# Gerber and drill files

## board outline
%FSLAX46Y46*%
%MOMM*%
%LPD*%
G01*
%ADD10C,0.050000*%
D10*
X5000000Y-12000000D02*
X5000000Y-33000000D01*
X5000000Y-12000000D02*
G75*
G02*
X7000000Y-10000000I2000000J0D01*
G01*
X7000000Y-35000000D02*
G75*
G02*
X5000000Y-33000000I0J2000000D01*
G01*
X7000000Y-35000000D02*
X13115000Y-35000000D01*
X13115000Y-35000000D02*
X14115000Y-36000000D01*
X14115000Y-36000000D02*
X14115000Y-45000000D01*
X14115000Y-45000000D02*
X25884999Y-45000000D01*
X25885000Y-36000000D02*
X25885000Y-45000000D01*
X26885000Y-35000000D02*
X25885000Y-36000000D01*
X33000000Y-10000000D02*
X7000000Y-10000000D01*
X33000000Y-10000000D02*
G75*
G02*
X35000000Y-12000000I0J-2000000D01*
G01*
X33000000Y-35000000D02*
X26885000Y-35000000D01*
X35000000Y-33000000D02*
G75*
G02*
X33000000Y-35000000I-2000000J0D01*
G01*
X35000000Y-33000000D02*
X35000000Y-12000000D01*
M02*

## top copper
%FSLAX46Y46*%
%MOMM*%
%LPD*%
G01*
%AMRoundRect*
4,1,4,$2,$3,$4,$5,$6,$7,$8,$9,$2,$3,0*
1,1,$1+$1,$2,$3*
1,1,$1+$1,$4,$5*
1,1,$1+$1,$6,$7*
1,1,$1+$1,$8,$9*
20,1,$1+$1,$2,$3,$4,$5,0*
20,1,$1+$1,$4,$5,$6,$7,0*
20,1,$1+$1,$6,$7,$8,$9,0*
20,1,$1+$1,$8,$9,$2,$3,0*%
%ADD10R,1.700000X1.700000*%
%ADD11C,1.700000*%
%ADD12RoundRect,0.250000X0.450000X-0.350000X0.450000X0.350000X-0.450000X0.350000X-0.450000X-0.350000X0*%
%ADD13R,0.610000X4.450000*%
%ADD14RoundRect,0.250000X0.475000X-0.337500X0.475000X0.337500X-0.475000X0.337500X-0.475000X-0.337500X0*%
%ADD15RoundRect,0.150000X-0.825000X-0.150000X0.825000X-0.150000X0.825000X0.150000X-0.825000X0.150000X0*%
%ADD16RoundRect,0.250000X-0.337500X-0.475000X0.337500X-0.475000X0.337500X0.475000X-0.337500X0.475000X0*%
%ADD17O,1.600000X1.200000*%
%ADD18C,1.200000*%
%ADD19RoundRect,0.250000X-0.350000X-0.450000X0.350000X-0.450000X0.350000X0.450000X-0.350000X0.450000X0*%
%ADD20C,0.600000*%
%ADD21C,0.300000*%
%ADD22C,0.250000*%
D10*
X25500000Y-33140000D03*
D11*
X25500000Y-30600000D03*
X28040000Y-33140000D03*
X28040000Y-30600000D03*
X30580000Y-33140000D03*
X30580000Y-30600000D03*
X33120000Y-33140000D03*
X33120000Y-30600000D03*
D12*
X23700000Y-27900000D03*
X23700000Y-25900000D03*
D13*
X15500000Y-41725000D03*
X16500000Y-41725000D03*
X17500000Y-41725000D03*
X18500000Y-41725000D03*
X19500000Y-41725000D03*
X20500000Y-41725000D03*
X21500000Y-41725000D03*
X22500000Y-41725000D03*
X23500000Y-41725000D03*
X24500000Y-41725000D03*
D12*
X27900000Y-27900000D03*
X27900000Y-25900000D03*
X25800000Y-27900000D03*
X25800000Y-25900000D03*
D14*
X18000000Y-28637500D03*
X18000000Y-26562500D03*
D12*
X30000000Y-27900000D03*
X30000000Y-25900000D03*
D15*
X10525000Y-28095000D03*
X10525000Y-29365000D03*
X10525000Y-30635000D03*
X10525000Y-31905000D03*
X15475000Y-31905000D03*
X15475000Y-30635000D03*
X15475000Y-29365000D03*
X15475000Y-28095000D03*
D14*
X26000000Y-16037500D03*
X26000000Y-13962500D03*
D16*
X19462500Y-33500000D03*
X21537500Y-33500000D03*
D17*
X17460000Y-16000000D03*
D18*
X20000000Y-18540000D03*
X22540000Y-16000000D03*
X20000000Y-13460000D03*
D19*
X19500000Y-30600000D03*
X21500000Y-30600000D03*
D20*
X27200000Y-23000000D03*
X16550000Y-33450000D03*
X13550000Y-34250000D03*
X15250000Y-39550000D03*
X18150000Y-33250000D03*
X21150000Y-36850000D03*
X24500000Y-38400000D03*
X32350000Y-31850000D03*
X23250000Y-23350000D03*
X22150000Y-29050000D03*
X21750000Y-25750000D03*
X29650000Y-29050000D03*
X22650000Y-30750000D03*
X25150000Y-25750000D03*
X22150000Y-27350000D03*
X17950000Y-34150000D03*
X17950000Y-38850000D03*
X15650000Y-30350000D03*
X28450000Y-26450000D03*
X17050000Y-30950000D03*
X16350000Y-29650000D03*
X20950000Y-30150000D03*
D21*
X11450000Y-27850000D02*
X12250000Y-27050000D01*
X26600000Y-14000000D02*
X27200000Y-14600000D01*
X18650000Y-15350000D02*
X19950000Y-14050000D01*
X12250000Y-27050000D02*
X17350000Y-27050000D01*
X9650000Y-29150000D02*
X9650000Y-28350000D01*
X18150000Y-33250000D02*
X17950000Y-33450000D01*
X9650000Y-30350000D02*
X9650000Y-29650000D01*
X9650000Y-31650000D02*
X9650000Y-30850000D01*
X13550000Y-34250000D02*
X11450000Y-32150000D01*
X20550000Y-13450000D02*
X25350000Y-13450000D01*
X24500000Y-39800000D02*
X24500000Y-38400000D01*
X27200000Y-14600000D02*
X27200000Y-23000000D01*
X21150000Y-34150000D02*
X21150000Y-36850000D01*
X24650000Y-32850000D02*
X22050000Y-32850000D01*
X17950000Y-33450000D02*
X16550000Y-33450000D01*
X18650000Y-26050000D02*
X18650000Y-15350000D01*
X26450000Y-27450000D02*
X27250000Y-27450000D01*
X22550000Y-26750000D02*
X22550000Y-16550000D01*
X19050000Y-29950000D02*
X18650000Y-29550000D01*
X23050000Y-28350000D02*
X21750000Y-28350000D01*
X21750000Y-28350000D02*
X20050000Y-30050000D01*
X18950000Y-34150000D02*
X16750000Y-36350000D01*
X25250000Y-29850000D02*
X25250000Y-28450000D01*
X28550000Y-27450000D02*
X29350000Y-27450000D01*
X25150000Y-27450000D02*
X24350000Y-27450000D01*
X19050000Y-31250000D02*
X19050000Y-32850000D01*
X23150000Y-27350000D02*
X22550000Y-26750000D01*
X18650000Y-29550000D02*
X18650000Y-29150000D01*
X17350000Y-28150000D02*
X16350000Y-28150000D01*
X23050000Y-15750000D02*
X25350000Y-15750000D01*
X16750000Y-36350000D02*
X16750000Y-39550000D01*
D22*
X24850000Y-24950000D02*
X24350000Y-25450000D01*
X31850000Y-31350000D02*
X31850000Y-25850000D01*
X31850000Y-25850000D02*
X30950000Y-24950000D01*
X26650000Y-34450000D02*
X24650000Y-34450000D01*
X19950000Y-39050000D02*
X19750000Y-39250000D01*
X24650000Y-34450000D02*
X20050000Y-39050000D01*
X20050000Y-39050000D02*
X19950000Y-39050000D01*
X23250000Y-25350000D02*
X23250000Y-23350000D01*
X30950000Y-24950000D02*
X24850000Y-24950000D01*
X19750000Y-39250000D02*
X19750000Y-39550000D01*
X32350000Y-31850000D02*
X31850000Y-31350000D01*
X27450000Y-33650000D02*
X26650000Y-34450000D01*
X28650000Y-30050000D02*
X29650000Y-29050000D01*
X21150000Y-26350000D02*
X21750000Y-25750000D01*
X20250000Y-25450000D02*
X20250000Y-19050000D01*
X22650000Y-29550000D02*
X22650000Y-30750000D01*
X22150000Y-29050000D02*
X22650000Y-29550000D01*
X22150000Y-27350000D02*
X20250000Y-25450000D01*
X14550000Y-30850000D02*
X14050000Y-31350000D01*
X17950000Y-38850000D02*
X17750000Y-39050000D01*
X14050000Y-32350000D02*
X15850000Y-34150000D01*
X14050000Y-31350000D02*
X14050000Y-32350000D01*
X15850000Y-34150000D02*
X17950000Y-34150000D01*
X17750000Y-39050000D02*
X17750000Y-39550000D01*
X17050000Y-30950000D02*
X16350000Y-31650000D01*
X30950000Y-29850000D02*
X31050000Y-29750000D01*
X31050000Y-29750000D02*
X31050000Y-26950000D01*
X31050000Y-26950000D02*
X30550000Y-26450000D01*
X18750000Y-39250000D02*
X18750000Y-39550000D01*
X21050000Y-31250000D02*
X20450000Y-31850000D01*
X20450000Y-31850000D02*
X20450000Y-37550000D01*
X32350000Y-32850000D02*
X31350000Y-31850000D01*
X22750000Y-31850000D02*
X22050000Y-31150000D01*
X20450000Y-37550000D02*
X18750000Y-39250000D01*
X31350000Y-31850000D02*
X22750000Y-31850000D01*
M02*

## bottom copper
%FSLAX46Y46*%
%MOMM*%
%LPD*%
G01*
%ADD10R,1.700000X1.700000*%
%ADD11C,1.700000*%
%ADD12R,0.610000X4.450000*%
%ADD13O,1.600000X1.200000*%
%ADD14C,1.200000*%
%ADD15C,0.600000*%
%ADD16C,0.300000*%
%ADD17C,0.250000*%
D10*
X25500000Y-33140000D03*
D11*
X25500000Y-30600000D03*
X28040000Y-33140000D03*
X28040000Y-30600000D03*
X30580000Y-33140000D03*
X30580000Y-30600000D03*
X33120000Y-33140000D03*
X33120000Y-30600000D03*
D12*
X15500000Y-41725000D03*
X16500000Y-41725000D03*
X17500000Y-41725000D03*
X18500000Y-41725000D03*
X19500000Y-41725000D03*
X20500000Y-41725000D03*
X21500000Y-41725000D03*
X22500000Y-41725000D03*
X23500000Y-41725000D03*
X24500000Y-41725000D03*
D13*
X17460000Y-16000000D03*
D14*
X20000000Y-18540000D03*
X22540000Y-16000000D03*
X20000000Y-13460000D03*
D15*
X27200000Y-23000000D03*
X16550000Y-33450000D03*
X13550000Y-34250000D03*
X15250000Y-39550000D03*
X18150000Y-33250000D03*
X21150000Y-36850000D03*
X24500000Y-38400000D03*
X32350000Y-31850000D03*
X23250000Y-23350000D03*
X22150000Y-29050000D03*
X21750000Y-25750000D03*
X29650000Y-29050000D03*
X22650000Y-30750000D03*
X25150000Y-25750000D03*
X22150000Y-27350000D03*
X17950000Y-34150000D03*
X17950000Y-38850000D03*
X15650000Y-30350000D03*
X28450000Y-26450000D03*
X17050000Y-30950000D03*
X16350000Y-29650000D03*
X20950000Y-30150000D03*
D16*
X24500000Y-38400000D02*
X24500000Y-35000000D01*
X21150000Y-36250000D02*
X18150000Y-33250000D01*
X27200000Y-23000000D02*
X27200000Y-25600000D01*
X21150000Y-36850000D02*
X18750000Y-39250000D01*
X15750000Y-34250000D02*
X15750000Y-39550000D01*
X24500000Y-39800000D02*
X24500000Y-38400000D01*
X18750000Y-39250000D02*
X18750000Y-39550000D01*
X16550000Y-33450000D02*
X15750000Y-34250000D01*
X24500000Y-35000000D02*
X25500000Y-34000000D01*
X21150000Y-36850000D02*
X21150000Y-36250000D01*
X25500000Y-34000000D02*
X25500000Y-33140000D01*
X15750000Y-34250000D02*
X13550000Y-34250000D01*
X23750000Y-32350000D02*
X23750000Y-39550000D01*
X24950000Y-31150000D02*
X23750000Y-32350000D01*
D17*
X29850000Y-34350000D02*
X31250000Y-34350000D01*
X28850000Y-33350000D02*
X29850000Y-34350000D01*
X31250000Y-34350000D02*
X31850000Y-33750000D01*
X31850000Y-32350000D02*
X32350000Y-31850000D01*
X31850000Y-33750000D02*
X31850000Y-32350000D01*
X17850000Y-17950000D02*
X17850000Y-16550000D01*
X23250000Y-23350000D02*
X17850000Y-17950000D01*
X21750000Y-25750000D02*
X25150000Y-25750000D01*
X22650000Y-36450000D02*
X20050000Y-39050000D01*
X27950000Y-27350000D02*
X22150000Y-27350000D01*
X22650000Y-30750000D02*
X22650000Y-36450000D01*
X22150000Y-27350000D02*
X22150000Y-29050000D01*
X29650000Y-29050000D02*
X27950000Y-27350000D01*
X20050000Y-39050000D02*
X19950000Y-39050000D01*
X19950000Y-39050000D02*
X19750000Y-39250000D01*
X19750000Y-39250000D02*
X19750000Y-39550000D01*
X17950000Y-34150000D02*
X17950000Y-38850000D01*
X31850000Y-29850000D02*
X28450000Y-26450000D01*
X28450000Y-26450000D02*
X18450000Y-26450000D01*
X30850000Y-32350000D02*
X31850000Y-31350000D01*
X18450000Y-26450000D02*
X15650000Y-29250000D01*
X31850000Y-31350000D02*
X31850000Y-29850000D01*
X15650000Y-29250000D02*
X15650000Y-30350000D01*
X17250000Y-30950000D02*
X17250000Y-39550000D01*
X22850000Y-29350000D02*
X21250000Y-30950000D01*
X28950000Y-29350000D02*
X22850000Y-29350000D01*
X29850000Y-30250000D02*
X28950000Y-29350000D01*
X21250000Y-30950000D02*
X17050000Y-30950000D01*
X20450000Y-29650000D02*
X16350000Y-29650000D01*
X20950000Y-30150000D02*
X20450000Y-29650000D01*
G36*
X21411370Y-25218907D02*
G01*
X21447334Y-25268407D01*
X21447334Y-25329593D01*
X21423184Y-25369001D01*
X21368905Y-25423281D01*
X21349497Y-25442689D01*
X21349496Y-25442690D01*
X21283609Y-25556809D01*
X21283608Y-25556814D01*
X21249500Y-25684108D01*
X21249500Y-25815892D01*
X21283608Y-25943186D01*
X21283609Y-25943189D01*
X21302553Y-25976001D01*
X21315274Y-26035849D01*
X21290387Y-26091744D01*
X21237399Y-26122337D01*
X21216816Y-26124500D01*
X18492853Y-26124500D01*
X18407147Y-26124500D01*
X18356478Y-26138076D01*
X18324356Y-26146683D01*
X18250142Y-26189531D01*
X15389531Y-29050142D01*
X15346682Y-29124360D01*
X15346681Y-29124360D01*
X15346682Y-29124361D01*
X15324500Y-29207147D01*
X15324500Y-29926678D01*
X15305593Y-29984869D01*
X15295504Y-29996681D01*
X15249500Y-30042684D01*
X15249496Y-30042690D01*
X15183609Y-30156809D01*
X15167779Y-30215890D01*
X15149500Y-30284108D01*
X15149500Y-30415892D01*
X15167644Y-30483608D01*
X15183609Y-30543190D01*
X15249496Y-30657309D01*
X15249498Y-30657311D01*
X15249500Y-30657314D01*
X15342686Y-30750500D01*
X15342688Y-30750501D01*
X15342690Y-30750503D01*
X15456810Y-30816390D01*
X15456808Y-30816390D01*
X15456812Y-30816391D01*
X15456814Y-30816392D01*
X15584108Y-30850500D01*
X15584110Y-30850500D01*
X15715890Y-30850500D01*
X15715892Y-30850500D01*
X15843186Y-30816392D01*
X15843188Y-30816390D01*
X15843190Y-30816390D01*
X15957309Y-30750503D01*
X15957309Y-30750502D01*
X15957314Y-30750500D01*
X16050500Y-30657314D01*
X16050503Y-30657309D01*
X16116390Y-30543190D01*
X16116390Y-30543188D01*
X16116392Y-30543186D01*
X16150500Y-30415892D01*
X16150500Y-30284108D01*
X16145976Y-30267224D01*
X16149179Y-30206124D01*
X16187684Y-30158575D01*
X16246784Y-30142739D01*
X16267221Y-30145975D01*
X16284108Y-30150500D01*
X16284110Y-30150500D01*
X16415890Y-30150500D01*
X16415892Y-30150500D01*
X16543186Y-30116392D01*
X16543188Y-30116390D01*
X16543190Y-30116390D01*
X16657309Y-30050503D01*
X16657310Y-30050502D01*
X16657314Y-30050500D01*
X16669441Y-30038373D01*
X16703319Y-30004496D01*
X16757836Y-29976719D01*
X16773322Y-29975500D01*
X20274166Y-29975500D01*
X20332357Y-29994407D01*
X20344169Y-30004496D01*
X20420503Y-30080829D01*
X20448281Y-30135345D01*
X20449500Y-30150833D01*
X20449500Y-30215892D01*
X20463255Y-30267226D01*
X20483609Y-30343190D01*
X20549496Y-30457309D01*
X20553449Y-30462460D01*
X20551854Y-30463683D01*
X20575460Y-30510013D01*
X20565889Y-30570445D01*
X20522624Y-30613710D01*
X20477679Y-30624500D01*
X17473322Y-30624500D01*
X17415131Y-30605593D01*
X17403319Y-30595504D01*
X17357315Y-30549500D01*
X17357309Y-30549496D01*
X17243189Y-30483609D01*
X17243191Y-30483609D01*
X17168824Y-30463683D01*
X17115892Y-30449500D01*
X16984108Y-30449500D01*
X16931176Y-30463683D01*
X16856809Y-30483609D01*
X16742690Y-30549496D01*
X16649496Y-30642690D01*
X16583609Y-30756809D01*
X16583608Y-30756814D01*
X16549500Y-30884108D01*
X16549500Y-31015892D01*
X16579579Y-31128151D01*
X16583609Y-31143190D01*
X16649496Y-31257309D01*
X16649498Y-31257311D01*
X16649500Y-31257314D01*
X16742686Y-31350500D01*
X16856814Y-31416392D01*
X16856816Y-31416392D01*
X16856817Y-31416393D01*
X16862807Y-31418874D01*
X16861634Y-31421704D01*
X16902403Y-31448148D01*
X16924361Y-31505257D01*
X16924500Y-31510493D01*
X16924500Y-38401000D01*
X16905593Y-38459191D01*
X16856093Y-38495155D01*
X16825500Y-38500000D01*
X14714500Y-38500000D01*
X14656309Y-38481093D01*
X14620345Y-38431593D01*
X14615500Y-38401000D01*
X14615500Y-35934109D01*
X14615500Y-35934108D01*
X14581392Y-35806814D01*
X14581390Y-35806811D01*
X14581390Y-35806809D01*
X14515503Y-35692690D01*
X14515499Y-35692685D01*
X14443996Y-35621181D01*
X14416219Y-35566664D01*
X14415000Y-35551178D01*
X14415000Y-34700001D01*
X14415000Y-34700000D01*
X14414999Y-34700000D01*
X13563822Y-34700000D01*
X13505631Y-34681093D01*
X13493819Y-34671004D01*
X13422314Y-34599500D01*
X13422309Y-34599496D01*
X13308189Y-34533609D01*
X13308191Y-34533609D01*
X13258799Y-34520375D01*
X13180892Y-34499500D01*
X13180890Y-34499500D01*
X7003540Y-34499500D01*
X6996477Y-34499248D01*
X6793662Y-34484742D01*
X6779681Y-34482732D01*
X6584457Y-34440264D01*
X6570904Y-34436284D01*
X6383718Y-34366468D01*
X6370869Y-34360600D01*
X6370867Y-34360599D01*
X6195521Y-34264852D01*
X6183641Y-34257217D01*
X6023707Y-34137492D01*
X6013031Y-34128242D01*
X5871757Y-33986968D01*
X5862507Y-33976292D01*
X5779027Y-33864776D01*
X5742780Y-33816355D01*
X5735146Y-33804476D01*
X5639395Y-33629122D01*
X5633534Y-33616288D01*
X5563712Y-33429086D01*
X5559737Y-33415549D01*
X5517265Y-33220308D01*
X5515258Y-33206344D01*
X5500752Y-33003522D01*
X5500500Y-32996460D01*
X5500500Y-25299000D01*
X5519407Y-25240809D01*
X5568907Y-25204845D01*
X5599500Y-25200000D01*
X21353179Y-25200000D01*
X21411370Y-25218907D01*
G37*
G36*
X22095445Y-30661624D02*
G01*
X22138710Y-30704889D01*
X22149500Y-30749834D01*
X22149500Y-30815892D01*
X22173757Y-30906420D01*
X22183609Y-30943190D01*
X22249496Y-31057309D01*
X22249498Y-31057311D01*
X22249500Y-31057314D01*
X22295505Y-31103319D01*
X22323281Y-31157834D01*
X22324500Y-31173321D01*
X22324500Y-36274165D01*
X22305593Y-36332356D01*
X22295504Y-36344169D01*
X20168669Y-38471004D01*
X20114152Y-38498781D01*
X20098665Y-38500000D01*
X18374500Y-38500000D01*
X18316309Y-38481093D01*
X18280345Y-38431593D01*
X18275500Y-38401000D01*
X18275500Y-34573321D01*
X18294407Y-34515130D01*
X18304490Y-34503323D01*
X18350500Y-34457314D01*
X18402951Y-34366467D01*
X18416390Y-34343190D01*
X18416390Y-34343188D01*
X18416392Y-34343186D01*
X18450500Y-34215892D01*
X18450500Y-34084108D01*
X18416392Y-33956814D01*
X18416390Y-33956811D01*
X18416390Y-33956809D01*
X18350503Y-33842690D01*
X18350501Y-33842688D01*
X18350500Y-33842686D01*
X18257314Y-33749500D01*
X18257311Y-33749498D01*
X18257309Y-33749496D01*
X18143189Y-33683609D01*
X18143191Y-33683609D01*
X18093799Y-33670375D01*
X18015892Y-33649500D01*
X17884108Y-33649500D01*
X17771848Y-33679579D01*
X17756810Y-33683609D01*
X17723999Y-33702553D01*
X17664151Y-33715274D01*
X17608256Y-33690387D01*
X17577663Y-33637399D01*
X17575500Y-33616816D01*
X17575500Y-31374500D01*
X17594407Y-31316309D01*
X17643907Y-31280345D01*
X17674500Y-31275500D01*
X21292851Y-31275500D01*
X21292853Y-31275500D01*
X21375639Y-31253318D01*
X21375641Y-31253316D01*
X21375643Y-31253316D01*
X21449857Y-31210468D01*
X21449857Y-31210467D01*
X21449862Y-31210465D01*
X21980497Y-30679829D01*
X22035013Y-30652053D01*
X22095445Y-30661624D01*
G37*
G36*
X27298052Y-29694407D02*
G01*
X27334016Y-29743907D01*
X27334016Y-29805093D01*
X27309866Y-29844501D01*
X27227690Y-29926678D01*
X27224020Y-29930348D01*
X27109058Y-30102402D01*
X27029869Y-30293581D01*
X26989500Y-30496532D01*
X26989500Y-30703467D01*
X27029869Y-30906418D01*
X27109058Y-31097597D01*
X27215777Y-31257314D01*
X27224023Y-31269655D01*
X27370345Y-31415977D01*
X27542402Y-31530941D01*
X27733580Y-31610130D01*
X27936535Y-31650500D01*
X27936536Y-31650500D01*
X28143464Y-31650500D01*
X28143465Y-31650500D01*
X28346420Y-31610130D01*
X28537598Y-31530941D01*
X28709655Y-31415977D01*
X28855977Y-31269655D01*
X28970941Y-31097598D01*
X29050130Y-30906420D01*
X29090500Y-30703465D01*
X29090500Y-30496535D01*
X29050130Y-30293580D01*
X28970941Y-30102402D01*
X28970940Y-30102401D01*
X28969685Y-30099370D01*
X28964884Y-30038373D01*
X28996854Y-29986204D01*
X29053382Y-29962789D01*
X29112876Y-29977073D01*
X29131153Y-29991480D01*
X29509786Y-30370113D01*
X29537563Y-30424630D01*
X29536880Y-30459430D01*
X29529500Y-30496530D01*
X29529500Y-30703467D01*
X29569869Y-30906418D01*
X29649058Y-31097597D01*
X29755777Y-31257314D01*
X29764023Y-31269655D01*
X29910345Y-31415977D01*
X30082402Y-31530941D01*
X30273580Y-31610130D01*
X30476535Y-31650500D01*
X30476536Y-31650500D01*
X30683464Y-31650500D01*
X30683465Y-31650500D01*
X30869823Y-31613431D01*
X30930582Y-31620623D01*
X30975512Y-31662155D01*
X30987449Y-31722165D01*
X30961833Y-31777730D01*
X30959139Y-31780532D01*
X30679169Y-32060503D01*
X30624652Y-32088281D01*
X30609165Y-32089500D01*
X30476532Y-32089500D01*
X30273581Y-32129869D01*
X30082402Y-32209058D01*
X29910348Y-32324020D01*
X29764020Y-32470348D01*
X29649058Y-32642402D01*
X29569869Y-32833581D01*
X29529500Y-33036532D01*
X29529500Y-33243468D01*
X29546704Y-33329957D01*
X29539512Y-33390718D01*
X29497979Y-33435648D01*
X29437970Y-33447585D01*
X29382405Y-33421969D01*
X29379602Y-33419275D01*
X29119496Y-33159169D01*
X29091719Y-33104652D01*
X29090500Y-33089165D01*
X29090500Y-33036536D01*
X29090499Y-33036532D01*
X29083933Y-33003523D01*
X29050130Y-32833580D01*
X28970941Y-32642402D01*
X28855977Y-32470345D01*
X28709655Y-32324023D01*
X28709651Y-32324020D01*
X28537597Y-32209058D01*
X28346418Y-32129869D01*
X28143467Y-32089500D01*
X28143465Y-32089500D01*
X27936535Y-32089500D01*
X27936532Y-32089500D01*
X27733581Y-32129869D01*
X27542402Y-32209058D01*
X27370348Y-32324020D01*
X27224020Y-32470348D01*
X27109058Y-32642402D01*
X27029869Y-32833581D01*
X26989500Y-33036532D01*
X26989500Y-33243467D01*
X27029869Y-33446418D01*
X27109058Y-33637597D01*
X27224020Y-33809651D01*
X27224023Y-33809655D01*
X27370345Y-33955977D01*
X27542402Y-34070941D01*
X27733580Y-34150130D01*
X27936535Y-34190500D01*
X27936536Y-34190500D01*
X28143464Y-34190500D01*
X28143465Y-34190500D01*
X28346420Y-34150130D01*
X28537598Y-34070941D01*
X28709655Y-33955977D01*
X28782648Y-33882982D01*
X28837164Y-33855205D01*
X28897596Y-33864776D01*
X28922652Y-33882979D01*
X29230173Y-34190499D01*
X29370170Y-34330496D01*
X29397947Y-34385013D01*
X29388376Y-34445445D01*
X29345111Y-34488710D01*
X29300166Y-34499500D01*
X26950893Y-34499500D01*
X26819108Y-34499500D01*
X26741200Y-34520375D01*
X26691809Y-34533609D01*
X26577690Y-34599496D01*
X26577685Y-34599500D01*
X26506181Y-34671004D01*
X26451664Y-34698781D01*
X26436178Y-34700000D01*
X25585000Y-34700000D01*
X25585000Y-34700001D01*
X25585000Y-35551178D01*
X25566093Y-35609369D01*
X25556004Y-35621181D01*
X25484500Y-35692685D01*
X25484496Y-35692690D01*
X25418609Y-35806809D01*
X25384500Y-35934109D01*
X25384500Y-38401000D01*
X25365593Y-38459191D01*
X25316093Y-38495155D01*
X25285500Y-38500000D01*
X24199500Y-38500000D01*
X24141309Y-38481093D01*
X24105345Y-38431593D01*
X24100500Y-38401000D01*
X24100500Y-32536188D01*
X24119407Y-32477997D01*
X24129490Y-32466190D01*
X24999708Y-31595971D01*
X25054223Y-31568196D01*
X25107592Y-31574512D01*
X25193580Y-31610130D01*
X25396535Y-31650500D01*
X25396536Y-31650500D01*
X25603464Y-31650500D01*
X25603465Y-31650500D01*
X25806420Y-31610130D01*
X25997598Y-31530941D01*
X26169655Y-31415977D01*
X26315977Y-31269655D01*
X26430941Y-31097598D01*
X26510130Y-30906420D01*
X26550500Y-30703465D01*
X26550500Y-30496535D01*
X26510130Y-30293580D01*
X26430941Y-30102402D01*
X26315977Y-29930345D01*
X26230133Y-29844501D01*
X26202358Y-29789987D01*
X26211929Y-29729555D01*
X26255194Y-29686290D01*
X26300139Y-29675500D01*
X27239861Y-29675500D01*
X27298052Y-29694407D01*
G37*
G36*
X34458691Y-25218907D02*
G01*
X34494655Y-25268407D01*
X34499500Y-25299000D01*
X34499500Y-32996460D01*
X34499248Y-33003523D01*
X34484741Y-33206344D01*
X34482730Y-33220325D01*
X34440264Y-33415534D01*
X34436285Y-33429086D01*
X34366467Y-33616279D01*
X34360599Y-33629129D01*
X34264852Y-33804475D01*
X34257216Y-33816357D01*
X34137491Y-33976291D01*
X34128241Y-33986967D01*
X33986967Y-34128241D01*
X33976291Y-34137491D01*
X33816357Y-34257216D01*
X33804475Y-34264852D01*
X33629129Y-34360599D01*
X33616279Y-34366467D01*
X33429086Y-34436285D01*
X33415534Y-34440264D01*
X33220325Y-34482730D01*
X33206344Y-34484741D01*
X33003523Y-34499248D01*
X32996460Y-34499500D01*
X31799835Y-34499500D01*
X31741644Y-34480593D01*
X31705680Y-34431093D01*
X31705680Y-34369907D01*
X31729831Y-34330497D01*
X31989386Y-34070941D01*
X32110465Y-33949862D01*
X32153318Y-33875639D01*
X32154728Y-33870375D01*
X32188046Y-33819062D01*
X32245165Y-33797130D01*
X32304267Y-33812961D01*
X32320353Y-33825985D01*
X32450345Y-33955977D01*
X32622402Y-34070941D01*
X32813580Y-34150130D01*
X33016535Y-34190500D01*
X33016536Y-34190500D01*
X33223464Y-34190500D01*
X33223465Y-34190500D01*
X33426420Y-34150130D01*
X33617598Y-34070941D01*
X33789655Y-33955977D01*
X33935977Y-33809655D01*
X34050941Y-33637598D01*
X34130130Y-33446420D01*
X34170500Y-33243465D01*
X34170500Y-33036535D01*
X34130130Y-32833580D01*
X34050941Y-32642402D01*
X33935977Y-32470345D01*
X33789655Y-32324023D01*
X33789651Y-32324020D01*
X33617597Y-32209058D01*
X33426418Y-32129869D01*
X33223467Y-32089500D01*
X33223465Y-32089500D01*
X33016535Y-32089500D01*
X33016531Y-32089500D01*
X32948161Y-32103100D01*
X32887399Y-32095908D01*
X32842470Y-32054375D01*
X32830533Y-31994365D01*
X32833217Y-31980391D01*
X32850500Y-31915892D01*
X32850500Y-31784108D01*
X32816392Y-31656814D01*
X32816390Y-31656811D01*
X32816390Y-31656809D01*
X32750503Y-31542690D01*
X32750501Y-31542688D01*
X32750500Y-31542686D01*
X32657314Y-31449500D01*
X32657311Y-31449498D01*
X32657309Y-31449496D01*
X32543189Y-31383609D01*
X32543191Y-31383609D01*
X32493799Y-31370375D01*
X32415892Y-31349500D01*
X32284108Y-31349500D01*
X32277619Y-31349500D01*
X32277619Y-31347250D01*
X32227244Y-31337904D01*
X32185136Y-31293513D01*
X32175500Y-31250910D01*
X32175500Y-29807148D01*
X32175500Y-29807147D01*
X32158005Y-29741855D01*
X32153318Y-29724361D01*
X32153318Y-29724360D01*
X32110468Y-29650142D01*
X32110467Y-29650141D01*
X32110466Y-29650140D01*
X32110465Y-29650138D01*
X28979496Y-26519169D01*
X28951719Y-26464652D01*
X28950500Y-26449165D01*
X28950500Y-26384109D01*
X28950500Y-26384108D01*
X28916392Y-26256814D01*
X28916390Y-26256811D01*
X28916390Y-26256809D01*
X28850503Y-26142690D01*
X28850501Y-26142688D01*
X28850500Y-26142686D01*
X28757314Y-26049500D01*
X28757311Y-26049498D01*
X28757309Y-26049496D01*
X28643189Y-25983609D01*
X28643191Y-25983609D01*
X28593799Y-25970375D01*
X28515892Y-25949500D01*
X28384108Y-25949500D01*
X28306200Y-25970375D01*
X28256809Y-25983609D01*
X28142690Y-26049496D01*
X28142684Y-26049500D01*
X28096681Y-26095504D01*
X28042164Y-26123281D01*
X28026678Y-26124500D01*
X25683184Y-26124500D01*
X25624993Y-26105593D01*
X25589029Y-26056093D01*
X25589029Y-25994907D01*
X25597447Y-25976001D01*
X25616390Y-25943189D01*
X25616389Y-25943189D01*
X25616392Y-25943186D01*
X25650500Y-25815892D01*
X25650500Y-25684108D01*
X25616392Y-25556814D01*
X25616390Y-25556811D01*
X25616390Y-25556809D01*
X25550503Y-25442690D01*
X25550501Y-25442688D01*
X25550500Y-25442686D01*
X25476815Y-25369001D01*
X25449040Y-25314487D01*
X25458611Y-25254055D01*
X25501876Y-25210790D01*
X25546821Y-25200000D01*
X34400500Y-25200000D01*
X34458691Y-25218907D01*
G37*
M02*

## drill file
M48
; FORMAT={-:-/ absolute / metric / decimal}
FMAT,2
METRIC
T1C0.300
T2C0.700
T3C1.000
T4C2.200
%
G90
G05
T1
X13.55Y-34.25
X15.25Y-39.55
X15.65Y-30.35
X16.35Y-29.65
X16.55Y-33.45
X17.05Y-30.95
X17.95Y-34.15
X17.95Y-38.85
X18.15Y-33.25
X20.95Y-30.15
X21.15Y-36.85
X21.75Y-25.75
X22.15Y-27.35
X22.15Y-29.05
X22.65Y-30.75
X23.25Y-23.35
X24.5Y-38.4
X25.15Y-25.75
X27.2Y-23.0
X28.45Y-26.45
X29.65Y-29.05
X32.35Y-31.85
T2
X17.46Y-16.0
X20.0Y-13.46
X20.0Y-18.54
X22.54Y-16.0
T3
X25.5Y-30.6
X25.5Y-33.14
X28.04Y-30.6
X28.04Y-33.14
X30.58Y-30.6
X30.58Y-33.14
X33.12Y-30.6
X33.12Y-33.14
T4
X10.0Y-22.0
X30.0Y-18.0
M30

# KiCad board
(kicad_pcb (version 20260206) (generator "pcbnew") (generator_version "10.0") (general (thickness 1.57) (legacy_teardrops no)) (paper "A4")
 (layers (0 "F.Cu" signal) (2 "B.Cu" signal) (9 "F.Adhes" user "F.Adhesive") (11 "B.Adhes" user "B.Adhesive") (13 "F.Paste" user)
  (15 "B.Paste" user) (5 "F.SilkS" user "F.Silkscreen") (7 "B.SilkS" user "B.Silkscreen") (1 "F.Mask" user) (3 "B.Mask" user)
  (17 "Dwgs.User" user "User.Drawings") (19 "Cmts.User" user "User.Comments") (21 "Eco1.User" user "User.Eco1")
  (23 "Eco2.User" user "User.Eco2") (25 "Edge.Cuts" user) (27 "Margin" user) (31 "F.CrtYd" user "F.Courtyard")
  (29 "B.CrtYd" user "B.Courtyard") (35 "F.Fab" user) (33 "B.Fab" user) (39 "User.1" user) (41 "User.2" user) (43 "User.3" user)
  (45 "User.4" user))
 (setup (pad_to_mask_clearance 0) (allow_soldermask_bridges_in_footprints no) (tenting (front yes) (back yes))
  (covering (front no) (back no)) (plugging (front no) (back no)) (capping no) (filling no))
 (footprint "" (layer "F.Cu") (at 30 18)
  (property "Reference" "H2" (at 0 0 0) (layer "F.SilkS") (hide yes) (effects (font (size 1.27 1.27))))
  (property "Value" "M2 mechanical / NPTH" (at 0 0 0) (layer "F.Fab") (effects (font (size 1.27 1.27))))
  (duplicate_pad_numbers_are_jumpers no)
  (pad "" np_thru_hole circle (at 0 0) (size 2.2 2.2) (drill 2.2) (layers "*.Cu" "*.Mask")))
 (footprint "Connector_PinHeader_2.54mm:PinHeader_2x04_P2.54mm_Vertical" (layer "F.Cu") (at 25.5 33.14 90)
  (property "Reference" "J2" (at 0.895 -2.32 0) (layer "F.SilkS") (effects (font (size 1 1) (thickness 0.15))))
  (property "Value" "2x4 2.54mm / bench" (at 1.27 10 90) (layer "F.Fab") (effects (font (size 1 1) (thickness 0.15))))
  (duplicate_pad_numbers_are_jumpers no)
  (pad "1" thru_hole rect (at 0 0 90) (size 1.7 1.7) (drill 1) (layers "*.Cu" "*.Mask") (remove_unused_layers no) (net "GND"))
  (pad "2" thru_hole circle (at 2.54 0 90) (size 1.7 1.7) (drill 1) (layers "*.Cu" "*.Mask") (remove_unused_layers no) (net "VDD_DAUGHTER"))
  (pad "3" thru_hole circle (at 0 2.54 90) (size 1.7 1.7) (drill 1) (layers "*.Cu" "*.Mask") (remove_unused_layers no) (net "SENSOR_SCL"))
  (pad "4" thru_hole circle (at 2.54 2.54 90) (size 1.7 1.7) (drill 1) (layers "*.Cu" "*.Mask") (remove_unused_layers no) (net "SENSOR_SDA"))
  (pad "5" thru_hole circle (at 0 5.08 90) (size 1.7 1.7) (drill 1) (layers "*.Cu" "*.Mask") (remove_unused_layers no) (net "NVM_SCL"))
  (pad "6" thru_hole circle (at 2.54 5.08 90) (size 1.7 1.7) (drill 1) (layers "*.Cu" "*.Mask") (remove_unused_layers no) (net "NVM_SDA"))
  (pad "7" thru_hole circle (at 0 7.62 90) (size 1.7 1.7) (drill 1) (layers "*.Cu" "*.Mask") (remove_unused_layers no) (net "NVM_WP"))
  (pad "8" thru_hole circle (at 2.54 7.62 90) (size 1.7 1.7) (drill 1) (layers "*.Cu" "*.Mask") (remove_unused_layers no) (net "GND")))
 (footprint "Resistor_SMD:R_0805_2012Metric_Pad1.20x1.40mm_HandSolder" (layer "F.Cu") (at 23.7 26.9 90)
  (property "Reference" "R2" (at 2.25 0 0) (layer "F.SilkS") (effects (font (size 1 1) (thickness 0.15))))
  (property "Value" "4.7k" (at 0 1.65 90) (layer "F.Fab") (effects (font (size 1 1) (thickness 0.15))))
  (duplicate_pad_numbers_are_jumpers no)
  (pad "1" smd roundrect (at -1 0 90) (size 1.2 1.4) (layers "F.Cu" "F.Mask" "F.Paste") (roundrect_rratio 0.208333) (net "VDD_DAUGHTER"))
  (pad "2" smd roundrect (at 1 0 90) (size 1.2 1.4) (layers "F.Cu" "F.Mask" "F.Paste") (roundrect_rratio 0.208333) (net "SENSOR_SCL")))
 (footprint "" (layer "F.Cu") (at 10 22)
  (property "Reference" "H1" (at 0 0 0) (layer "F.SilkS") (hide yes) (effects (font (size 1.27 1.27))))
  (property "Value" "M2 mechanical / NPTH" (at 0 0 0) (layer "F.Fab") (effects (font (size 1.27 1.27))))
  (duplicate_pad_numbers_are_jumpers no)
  (pad "" np_thru_hole circle (at 0 0) (size 2.2 2.2) (drill 2.2) (layers "*.Cu" "*.Mask")))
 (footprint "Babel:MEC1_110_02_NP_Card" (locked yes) (layer "F.Cu") (at 20 45)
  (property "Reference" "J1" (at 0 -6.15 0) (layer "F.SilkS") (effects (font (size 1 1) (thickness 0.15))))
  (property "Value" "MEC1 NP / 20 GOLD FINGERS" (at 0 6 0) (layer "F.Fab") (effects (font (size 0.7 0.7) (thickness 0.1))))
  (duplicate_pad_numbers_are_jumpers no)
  (pad "1" smd rect (at -4.5 -3.275) (size 0.61 4.45) (layers "F.Cu" "F.Mask") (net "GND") (solder_mask_margin 0.05))
  (pad "2" smd rect (at -4.5 -3.275) (size 0.61 4.45) (layers "B.Cu" "B.Mask") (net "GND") (solder_mask_margin 0.05))
  (pad "3" smd rect (at -3.5 -3.275) (size 0.61 4.45) (layers "F.Cu" "F.Mask") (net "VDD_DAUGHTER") (solder_mask_margin 0.05))
  (pad "4" smd rect (at -3.5 -3.275) (size 0.61 4.45) (layers "B.Cu" "B.Mask") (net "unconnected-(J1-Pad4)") (solder_mask_margin 0.05))
  (pad "5" smd rect (at -2.5 -3.275) (size 0.61 4.45) (layers "F.Cu" "F.Mask") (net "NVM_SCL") (solder_mask_margin 0.05))
  (pad "6" smd rect (at -2.5 -3.275) (size 0.61 4.45) (layers "B.Cu" "B.Mask") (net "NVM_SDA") (solder_mask_margin 0.05))
  (pad "7" smd rect (at -1.5 -3.275) (size 0.61 4.45) (layers "F.Cu" "F.Mask") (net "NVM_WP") (solder_mask_margin 0.05))
  (pad "8" smd rect (at -1.5 -3.275) (size 0.61 4.45) (layers "B.Cu" "B.Mask") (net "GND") (solder_mask_margin 0.05))
  (pad "9" smd rect (at -0.5 -3.275) (size 0.61 4.45) (layers "F.Cu" "F.Mask") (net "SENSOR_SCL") (solder_mask_margin 0.05))
  (pad "10" smd rect (at -0.5 -3.275) (size 0.61 4.45) (layers "B.Cu" "B.Mask") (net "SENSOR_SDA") (solder_mask_margin 0.05))
  (pad "11" smd rect (at 0.5 -3.275) (size 0.61 4.45) (layers "F.Cu" "F.Mask") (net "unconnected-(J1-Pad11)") (solder_mask_margin 0.05))
  (pad "12" smd rect (at 0.5 -3.275) (size 0.61 4.45) (layers "B.Cu" "B.Mask") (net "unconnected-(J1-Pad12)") (solder_mask_margin 0.05))
  (pad "13" smd rect (at 1.5 -3.275) (size 0.61 4.45) (layers "F.Cu" "F.Mask") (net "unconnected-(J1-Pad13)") (solder_mask_margin 0.05))
  (pad "14" smd rect (at 1.5 -3.275) (size 0.61 4.45) (layers "B.Cu" "B.Mask") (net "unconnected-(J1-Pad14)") (solder_mask_margin 0.05))
  (pad "15" smd rect (at 2.5 -3.275) (size 0.61 4.45) (layers "F.Cu" "F.Mask") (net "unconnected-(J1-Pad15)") (solder_mask_margin 0.05))
  (pad "16" smd rect (at 2.5 -3.275) (size 0.61 4.45) (layers "B.Cu" "B.Mask") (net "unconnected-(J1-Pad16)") (solder_mask_margin 0.05))
  (pad "17" smd rect (at 3.5 -3.275) (size 0.61 4.45) (layers "F.Cu" "F.Mask") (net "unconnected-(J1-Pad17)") (solder_mask_margin 0.05))
  (pad "18" smd rect (at 3.5 -3.275) (size 0.61 4.45) (layers "B.Cu" "B.Mask") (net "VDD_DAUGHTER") (solder_mask_margin 0.05))
  (pad "19" smd rect (at 4.5 -3.275) (size 0.61 4.45) (layers "F.Cu" "F.Mask") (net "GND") (solder_mask_margin 0.05))
  (pad "20" smd rect (at 4.5 -3.275) (size 0.61 4.45) (layers "B.Cu" "B.Mask") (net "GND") (solder_mask_margin 0.05)))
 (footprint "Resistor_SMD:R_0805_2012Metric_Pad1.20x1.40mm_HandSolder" (layer "F.Cu") (at 27.9 26.9 90)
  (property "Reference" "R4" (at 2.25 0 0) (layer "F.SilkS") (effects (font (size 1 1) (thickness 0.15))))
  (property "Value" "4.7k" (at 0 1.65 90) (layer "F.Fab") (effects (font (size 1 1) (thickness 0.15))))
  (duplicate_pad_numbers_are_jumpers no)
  (pad "1" smd roundrect (at -1 0 90) (size 1.2 1.4) (layers "F.Cu" "F.Mask" "F.Paste") (roundrect_rratio 0.208333) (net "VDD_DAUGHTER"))
  (pad "2" smd roundrect (at 1 0 90) (size 1.2 1.4) (layers "F.Cu" "F.Mask" "F.Paste") (roundrect_rratio 0.208333) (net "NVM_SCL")))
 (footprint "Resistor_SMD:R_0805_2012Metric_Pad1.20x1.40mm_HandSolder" (layer "F.Cu") (at 25.8 26.9 90)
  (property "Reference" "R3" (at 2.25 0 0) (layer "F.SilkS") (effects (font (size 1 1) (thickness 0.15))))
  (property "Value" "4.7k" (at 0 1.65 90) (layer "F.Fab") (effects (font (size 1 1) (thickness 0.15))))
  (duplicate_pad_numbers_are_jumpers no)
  (pad "1" smd roundrect (at -1 0 90) (size 1.2 1.4) (layers "F.Cu" "F.Mask" "F.Paste") (roundrect_rratio 0.208333) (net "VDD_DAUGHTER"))
  (pad "2" smd roundrect (at 1 0 90) (size 1.2 1.4) (layers "F.Cu" "F.Mask" "F.Paste") (roundrect_rratio 0.208333) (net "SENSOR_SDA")))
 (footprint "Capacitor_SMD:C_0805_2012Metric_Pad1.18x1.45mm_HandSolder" (layer "F.Cu") (at 18 27.6 90)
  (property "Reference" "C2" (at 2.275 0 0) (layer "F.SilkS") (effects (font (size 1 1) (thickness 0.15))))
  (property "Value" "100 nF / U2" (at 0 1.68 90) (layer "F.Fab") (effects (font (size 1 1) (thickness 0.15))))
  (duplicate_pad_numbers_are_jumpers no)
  (pad "1" smd roundrect (at -1.0375 0 90) (size 1.175 1.45) (layers "F.Cu" "F.Mask" "F.Paste") (roundrect_rratio 0.212766)
   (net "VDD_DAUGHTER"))
  (pad "2" smd roundrect (at 1.0375 0 90) (size 1.175 1.45) (layers "F.Cu" "F.Mask" "F.Paste") (roundrect_rratio 0.212766) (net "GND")))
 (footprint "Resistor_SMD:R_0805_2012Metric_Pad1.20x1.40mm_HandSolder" (layer "F.Cu") (at 30 26.9 90)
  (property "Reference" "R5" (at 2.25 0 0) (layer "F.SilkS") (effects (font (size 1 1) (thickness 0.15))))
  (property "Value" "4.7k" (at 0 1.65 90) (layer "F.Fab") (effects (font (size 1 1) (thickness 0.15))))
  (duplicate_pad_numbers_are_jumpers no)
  (pad "1" smd roundrect (at -1 0 90) (size 1.2 1.4) (layers "F.Cu" "F.Mask" "F.Paste") (roundrect_rratio 0.208333) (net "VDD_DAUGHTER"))
  (pad "2" smd roundrect (at 1 0 90) (size 1.2 1.4) (layers "F.Cu" "F.Mask" "F.Paste") (roundrect_rratio 0.208333) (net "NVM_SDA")))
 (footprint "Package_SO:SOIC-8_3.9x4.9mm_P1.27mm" (layer "F.Cu") (at 13 30)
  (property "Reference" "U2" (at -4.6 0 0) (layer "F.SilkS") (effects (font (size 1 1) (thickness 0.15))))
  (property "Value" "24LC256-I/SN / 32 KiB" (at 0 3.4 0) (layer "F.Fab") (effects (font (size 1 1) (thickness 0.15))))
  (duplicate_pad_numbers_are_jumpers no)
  (pad "1" smd roundrect (at -2.475 -1.905) (size 1.95 0.6) (layers "F.Cu" "F.Mask" "F.Paste") (roundrect_rratio 0.25) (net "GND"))
  (pad "2" smd roundrect (at -2.475 -0.635) (size 1.95 0.6) (layers "F.Cu" "F.Mask" "F.Paste") (roundrect_rratio 0.25) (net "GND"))
  (pad "3" smd roundrect (at -2.475 0.635) (size 1.95 0.6) (layers "F.Cu" "F.Mask" "F.Paste") (roundrect_rratio 0.25) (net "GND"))
  (pad "4" smd roundrect (at -2.475 1.905) (size 1.95 0.6) (layers "F.Cu" "F.Mask" "F.Paste") (roundrect_rratio 0.25) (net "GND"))
  (pad "5" smd roundrect (at 2.475 1.905) (size 1.95 0.6) (layers "F.Cu" "F.Mask" "F.Paste") (roundrect_rratio 0.25) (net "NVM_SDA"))
  (pad "6" smd roundrect (at 2.475 0.635) (size 1.95 0.6) (layers "F.Cu" "F.Mask" "F.Paste") (roundrect_rratio 0.25) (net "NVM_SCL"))
  (pad "7" smd roundrect (at 2.475 -0.635) (size 1.95 0.6) (layers "F.Cu" "F.Mask" "F.Paste") (roundrect_rratio 0.25) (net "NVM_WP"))
  (pad "8" smd roundrect (at 2.475 -1.905) (size 1.95 0.6) (layers "F.Cu" "F.Mask" "F.Paste") (roundrect_rratio 0.25) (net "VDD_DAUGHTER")))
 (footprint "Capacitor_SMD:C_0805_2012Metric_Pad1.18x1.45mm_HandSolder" (layer "F.Cu") (at 26 15 90)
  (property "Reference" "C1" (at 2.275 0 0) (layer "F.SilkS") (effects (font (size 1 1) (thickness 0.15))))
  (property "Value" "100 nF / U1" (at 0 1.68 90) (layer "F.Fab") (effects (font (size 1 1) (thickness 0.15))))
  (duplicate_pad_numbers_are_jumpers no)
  (pad "1" smd roundrect (at -1.0375 0 90) (size 1.175 1.45) (layers "F.Cu" "F.Mask" "F.Paste") (roundrect_rratio 0.212766)
   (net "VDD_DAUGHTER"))
  (pad "2" smd roundrect (at 1.0375 0 90) (size 1.175 1.45) (layers "F.Cu" "F.Mask" "F.Paste") (roundrect_rratio 0.212766) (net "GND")))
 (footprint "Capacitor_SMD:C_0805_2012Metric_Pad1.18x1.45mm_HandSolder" (layer "F.Cu") (at 20.5 33.5)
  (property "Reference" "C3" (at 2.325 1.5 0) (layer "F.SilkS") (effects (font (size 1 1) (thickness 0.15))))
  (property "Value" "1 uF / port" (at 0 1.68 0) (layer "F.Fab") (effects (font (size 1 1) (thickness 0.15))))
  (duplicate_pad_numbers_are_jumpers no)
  (pad "1" smd roundrect (at -1.0375 0) (size 1.175 1.45) (layers "F.Cu" "F.Mask" "F.Paste") (roundrect_rratio 0.212766)
   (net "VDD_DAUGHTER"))
  (pad "2" smd roundrect (at 1.0375 0) (size 1.175 1.45) (layers "F.Cu" "F.Mask" "F.Paste") (roundrect_rratio 0.212766) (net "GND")))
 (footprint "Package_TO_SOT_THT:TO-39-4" (layer "F.Cu") (at 17.46 16)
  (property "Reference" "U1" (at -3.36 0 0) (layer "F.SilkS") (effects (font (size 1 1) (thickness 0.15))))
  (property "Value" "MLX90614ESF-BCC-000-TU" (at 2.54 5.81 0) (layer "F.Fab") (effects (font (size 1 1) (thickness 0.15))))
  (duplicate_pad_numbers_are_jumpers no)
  (pad "1" thru_hole oval (at 0 0) (size 1.6 1.2) (drill 0.7) (layers "*.Cu" "*.Mask") (remove_unused_layers no) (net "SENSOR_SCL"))
  (pad "2" thru_hole circle (at 2.54 2.54) (size 1.2 1.2) (drill 0.7) (layers "*.Cu" "*.Mask") (remove_unused_layers no) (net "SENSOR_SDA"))
  (pad "3" thru_hole circle (at 5.08 0) (size 1.2 1.2) (drill 0.7) (layers "*.Cu" "*.Mask") (remove_unused_layers no) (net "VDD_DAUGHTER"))
  (pad "4" thru_hole circle (at 2.54 -2.54) (size 1.2 1.2) (drill 0.7) (layers "*.Cu" "*.Mask") (remove_unused_layers no) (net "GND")))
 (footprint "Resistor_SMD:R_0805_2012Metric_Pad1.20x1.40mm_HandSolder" (layer "F.Cu") (at 20.5 30.6)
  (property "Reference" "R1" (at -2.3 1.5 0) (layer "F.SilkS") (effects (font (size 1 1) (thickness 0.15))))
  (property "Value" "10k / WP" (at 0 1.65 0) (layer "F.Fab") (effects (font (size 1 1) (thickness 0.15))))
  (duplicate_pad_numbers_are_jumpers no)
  (pad "1" smd roundrect (at -1 0) (size 1.2 1.4) (layers "F.Cu" "F.Mask" "F.Paste") (roundrect_rratio 0.208333) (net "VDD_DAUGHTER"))
  (pad "2" smd roundrect (at 1 0) (size 1.2 1.4) (layers "F.Cu" "F.Mask" "F.Paste") (roundrect_rratio 0.208333) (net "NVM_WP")))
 (gr_line (start 5 12) (end 5 33) (stroke (width 0.05) (type default)) (layer "Edge.Cuts"))
 (gr_arc (start 5 12) (mid 5.585786 10.585786) (end 7 10) (stroke (width 0.05) (type default)) (layer "Edge.Cuts"))
 (gr_arc (start 7 35) (mid 5.585786 34.414214) (end 5 33) (stroke (width 0.05) (type default)) (layer "Edge.Cuts"))
 (gr_line (start 7 35) (end 13.115 35) (stroke (width 0.05) (type default)) (layer "Edge.Cuts"))
 (gr_line (start 13.115 35) (end 14.115 36) (stroke (width 0.05) (type default)) (layer "Edge.Cuts"))
 (gr_line (start 14.115 36) (end 14.115 45) (stroke (width 0.05) (type default)) (layer "Edge.Cuts"))
 (gr_line (start 14.115 45) (end 25.884999 45) (stroke (width 0.05) (type default)) (layer "Edge.Cuts"))
 (gr_line (start 25.885 36) (end 25.885 45) (stroke (width 0.05) (type default)) (layer "Edge.Cuts"))
 (gr_line (start 26.885 35) (end 25.885 36) (stroke (width 0.05) (type default)) (layer "Edge.Cuts"))
 (gr_line (start 33 10) (end 7 10) (stroke (width 0.05) (type default)) (layer "Edge.Cuts"))
 (gr_arc (start 33 10) (mid 34.414214 10.585786) (end 35 12) (stroke (width 0.05) (type default)) (layer "Edge.Cuts"))
 (gr_line (start 33 35) (end 26.885 35) (stroke (width 0.05) (type default)) (layer "Edge.Cuts"))
 (gr_arc (start 35 33) (mid 34.414213 34.414213) (end 33 35) (stroke (width 0.05) (type default)) (layer "Edge.Cuts"))
 (gr_line (start 35 33) (end 35 12) (stroke (width 0.05) (type default)) (layer "Edge.Cuts"))
 (segment (start 11.45 27.85) (end 12.25 27.05) (width 0.3) (layer "F.Cu") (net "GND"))
 (segment (start 26.6 14) (end 27.2 14.6) (width 0.3) (layer "F.Cu") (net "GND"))
 (segment (start 18.65 15.35) (end 19.95 14.05) (width 0.3) (layer "F.Cu") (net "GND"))
 (segment (start 12.25 27.05) (end 17.35 27.05) (width 0.3) (layer "F.Cu") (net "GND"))
 (segment (start 9.65 29.15) (end 9.65 28.35) (width 0.3) (layer "F.Cu") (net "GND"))
 (segment (start 18.15 33.25) (end 17.95 33.45) (width 0.3) (layer "F.Cu") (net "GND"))
 (segment (start 9.65 30.35) (end 9.65 29.65) (width 0.3) (layer "F.Cu") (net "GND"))
 (segment (start 9.65 31.65) (end 9.65 30.85) (width 0.3) (layer "F.Cu") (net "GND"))
 (segment (start 13.55 34.25) (end 11.45 32.15) (width 0.3) (layer "F.Cu") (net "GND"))
 (segment (start 20.55 13.45) (end 25.35 13.45) (width 0.3) (layer "F.Cu") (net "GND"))
 (segment (start 24.5 39.8) (end 24.5 38.4) (width 0.3) (layer "F.Cu") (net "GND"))
 (segment (start 27.2 14.6) (end 27.2 23) (width 0.3) (layer "F.Cu") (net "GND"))
 (segment (start 21.15 34.15) (end 21.15 36.85) (width 0.3) (layer "F.Cu") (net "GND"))
 (segment (start 24.65 32.85) (end 22.05 32.85) (width 0.3) (layer "F.Cu") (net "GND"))
 (segment (start 17.95 33.45) (end 16.55 33.45) (width 0.3) (layer "F.Cu") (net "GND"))
 (segment (start 18.65 26.05) (end 18.65 15.35) (width 0.3) (layer "F.Cu") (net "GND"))
 (via (at 27.2 23) (size 0.6) (drill 0.3) (layers "F.Cu" "B.Cu") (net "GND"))
 (via (at 16.55 33.45) (size 0.6) (drill 0.3) (layers "F.Cu" "B.Cu") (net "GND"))
 (via (at 13.55 34.25) (size 0.6) (drill 0.3) (layers "F.Cu" "B.Cu") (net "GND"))
 (via (at 15.25 39.55) (size 0.6) (drill 0.3) (layers "F.Cu" "B.Cu") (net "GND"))
 (via (at 18.15 33.25) (size 0.6) (drill 0.3) (layers "F.Cu" "B.Cu") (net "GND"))
 (via (at 21.15 36.85) (size 0.6) (drill 0.3) (layers "F.Cu" "B.Cu") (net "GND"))
 (via (at 24.5 38.4) (size 0.6) (drill 0.3) (layers "F.Cu" "B.Cu") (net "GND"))
 (segment (start 24.5 38.4) (end 24.5 35) (width 0.3) (layer "B.Cu") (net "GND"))
 (segment (start 21.15 36.25) (end 18.15 33.25) (width 0.3) (layer "B.Cu") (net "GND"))
 (segment (start 27.2 23) (end 27.2 25.6) (width 0.3) (layer "B.Cu") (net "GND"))
 (segment (start 21.15 36.85) (end 18.75 39.25) (width 0.3) (layer "B.Cu") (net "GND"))
 (segment (start 15.75 34.25) (end 15.75 39.55) (width 0.3) (layer "B.Cu") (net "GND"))
 (segment (start 24.5 39.8) (end 24.5 38.4) (width 0.3) (layer "B.Cu") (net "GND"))
 (segment (start 18.75 39.25) (end 18.75 39.55) (width 0.3) (layer "B.Cu") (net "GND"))
 (segment (start 16.55 33.45) (end 15.75 34.25) (width 0.3) (layer "B.Cu") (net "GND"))
 (segment (start 24.5 35) (end 25.5 34) (width 0.3) (layer "B.Cu") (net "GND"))
 (segment (start 21.15 36.85) (end 21.15 36.25) (width 0.3) (layer "B.Cu") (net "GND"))
 (segment (start 25.5 34) (end 25.5 33.14) (width 0.3) (layer "B.Cu") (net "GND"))
 (segment (start 15.75 34.25) (end 13.55 34.25) (width 0.3) (layer "B.Cu") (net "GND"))
 (segment (start 26.45 27.45) (end 27.25 27.45) (width 0.3) (layer "F.Cu") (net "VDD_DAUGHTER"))
 (segment (start 22.55 26.75) (end 22.55 16.55) (width 0.3) (layer "F.Cu") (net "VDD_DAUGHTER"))
 (segment (start 19.05 29.95) (end 18.65 29.55) (width 0.3) (layer "F.Cu") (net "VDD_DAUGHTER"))
 (segment (start 23.05 28.35) (end 21.75 28.35) (width 0.3) (layer "F.Cu") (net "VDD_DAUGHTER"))
 (segment (start 21.75 28.35) (end 20.05 30.05) (width 0.3) (layer "F.Cu") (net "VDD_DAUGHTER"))
 (segment (start 18.95 34.15) (end 16.75 36.35) (width 0.3) (layer "F.Cu") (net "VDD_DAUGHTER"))
 (segment (start 25.25 29.85) (end 25.25 28.45) (width 0.3) (layer "F.Cu") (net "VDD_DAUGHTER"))
 (segment (start 28.55 27.45) (end 29.35 27.45) (width 0.3) (layer "F.Cu") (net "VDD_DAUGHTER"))
 (segment (start 25.15 27.45) (end 24.35 27.45) (width 0.3) (layer "F.Cu") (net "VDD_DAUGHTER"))
 (segment (start 19.05 31.25) (end 19.05 32.85) (width 0.3) (layer "F.Cu") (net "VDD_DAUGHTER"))
 (segment (start 23.15 27.35) (end 22.55 26.75) (width 0.3) (layer "F.Cu") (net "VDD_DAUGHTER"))
 (segment (start 18.65 29.55) (end 18.65 29.15) (width 0.3) (layer "F.Cu") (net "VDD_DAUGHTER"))
 (segment (start 17.35 28.15) (end 16.35 28.15) (width 0.3) (layer "F.Cu") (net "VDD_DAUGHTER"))
 (segment (start 23.05 15.75) (end 25.35 15.75) (width 0.3) (layer "F.Cu") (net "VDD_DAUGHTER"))
 (segment (start 16.75 36.35) (end 16.75 39.55) (width 0.3) (layer "F.Cu") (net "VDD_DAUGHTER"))
 (segment (start 23.75 32.35) (end 23.75 39.55) (width 0.3) (layer "B.Cu") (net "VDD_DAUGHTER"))
 (segment (start 24.95 31.15) (end 23.75 32.35) (width 0.3) (layer "B.Cu") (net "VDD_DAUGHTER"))
 (segment (start 24.85 24.95) (end 24.35 25.45) (width 0.25) (layer "F.Cu") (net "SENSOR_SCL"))
 (segment (start 31.85 31.35) (end 31.85 25.85) (width 0.25) (layer "F.Cu") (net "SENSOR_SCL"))
 (segment (start 31.85 25.85) (end 30.95 24.95) (width 0.25) (layer "F.Cu") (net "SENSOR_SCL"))
 (segment (start 26.65 34.45) (end 24.65 34.45) (width 0.25) (layer "F.Cu") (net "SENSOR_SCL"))
 (segment (start 19.95 39.05) (end 19.75 39.25) (width 0.25) (layer "F.Cu") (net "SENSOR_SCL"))
 (segment (start 24.65 34.45) (end 20.05 39.05) (width 0.25) (layer "F.Cu") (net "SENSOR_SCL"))
 (segment (start 20.05 39.05) (end 19.95 39.05) (width 0.25) (layer "F.Cu") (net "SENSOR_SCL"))
 (segment (start 23.25 25.35) (end 23.25 23.35) (width 0.25) (layer "F.Cu") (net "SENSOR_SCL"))
 (segment (start 30.95 24.95) (end 24.85 24.95) (width 0.25) (layer "F.Cu") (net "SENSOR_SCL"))
 (segment (start 19.75 39.25) (end 19.75 39.55) (width 0.25) (layer "F.Cu") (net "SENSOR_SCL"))
 (segment (start 32.35 31.85) (end 31.85 31.35) (width 0.25) (layer "F.Cu") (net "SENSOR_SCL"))
 (segment (start 27.45 33.65) (end 26.65 34.45) (width 0.25) (layer "F.Cu") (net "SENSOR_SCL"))
 (via (at 32.35 31.85) (size 0.6) (drill 0.3) (layers "F.Cu" "B.Cu") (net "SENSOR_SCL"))
 (via (at 23.25 23.35) (size 0.6) (drill 0.3) (layers "F.Cu" "B.Cu") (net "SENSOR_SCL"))
 (segment (start 29.85 34.35) (end 31.25 34.35) (width 0.25) (layer "B.Cu") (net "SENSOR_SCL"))
 (segment (start 28.85 33.35) (end 29.85 34.35) (width 0.25) (layer "B.Cu") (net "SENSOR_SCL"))
 (segment (start 31.25 34.35) (end 31.85 33.75) (width 0.25) (layer "B.Cu") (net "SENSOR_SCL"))
 (segment (start 31.85 32.35) (end 32.35 31.85) (width 0.25) (layer "B.Cu") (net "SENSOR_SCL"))
 (segment (start 31.85 33.75) (end 31.85 32.35) (width 0.25) (layer "B.Cu") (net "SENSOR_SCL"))
 (segment (start 17.85 17.95) (end 17.85 16.55) (width 0.25) (layer "B.Cu") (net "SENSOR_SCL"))
 (segment (start 23.25 23.35) (end 17.85 17.95) (width 0.25) (layer "B.Cu") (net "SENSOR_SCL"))
 (segment (start 28.65 30.05) (end 29.65 29.05) (width 0.25) (layer "F.Cu") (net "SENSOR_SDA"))
 (segment (start 21.15 26.35) (end 21.75 25.75) (width 0.25) (layer "F.Cu") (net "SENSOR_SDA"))
 (segment (start 20.25 25.45) (end 20.25 19.05) (width 0.25) (layer "F.Cu") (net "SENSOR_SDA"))
 (segment (start 22.65 29.55) (end 22.65 30.75) (width 0.25) (layer "F.Cu") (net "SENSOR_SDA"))
 (segment (start 22.15 29.05) (end 22.65 29.55) (width 0.25) (layer "F.Cu") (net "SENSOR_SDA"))
 (segment (start 22.15 27.35) (end 20.25 25.45) (width 0.25) (layer "F.Cu") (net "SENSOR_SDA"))
 (via (at 22.15 29.05) (size 0.6) (drill 0.3) (layers "F.Cu" "B.Cu") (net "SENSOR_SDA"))
 (via (at 21.75 25.75) (size 0.6) (drill 0.3) (layers "F.Cu" "B.Cu") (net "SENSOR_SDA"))
 (via (at 29.65 29.05) (size 0.6) (drill 0.3) (layers "F.Cu" "B.Cu") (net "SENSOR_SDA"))
 (via (at 22.65 30.75) (size 0.6) (drill 0.3) (layers "F.Cu" "B.Cu") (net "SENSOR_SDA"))
 (via (at 25.15 25.75) (size 0.6) (drill 0.3) (layers "F.Cu" "B.Cu") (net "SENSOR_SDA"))
 (via (at 22.15 27.35) (size 0.6) (drill 0.3) (layers "F.Cu" "B.Cu") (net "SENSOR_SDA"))
 (segment (start 21.75 25.75) (end 25.15 25.75) (width 0.25) (layer "B.Cu") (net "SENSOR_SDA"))
 (segment (start 22.65 36.45) (end 20.05 39.05) (width 0.25) (layer "B.Cu") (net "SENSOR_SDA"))
 (segment (start 27.95 27.35) (end 22.15 27.35) (width 0.25) (layer "B.Cu") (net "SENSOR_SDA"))
 (segment (start 22.65 30.75) (end 22.65 36.45) (width 0.25) (layer "B.Cu") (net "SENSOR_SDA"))
 (segment (start 22.15 27.35) (end 22.15 29.05) (width 0.25) (layer "B.Cu") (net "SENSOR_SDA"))
 (segment (start 29.65 29.05) (end 27.95 27.35) (width 0.25) (layer "B.Cu") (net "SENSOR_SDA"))
 (segment (start 20.05 39.05) (end 19.95 39.05) (width 0.25) (layer "B.Cu") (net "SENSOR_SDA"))
 (segment (start 19.95 39.05) (end 19.75 39.25) (width 0.25) (layer "B.Cu") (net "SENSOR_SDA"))
 (segment (start 19.75 39.25) (end 19.75 39.55) (width 0.25) (layer "B.Cu") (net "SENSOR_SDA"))
 (segment (start 14.55 30.85) (end 14.05 31.35) (width 0.25) (layer "F.Cu") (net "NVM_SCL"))
 (segment (start 17.95 38.85) (end 17.75 39.05) (width 0.25) (layer "F.Cu") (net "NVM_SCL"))
 (segment (start 14.05 32.35) (end 15.85 34.15) (width 0.25) (layer "F.Cu") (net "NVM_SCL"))
 (segment (start 14.05 31.35) (end 14.05 32.35) (width 0.25) (layer "F.Cu") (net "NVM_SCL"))
 (segment (start 15.85 34.15) (end 17.95 34.15) (width 0.25) (layer "F.Cu") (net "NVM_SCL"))
 (segment (start 17.75 39.05) (end 17.75 39.55) (width 0.25) (layer "F.Cu") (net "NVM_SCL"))
 (via (at 17.95 34.15) (size 0.6) (drill 0.3) (layers "F.Cu" "B.Cu") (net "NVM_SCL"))
 (via (at 17.95 38.85) (size 0.6) (drill 0.3) (layers "F.Cu" "B.Cu") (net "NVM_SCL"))
 (via (at 15.65 30.35) (size 0.6) (drill 0.3) (layers "F.Cu" "B.Cu") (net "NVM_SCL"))
 (via (at 28.45 26.45) (size 0.6) (drill 0.3) (layers "F.Cu" "B.Cu") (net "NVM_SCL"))
 (segment (start 17.95 34.15) (end 17.95 38.85) (width 0.25) (layer "B.Cu") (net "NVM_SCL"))
 (segment (start 31.85 29.85) (end 28.45 26.45) (width 0.25) (layer "B.Cu") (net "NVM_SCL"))
 (segment (start 28.45 26.45) (end 18.45 26.45) (width 0.25) (layer "B.Cu") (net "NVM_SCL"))
 (segment (start 30.85 32.35) (end 31.85 31.35) (width 0.25) (layer "B.Cu") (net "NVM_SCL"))
 (segment (start 18.45 26.45) (end 15.65 29.25) (width 0.25) (layer "B.Cu") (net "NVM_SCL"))
 (segment (start 31.85 31.35) (end 31.85 29.85) (width 0.25) (layer "B.Cu") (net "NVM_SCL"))
 (segment (start 15.65 29.25) (end 15.65 30.35) (width 0.25) (layer "B.Cu") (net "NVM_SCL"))
 (segment (start 17.05 30.95) (end 16.35 31.65) (width 0.25) (layer "F.Cu") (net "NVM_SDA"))
 (segment (start 30.95 29.85) (end 31.05 29.75) (width 0.25) (layer "F.Cu") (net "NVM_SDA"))
 (segment (start 31.05 29.75) (end 31.05 26.95) (width 0.25) (layer "F.Cu") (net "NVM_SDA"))
 (segment (start 31.05 26.95) (end 30.55 26.45) (width 0.25) (layer "F.Cu") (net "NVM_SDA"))
 (via (at 17.05 30.95) (size 0.6) (drill 0.3) (layers "F.Cu" "B.Cu") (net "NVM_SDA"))
 (segment (start 17.25 30.95) (end 17.25 39.55) (width 0.25) (layer "B.Cu") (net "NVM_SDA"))
 (segment (start 22.85 29.35) (end 21.25 30.95) (width 0.25) (layer "B.Cu") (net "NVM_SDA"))
 (segment (start 28.95 29.35) (end 22.85 29.35) (width 0.25) (layer "B.Cu") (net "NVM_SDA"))
 (segment (start 29.85 30.25) (end 28.95 29.35) (width 0.25) (layer "B.Cu") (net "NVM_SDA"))
 (segment (start 21.25 30.95) (end 17.05 30.95) (width 0.25) (layer "B.Cu") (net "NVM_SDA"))
 (segment (start 18.75 39.25) (end 18.75 39.55) (width 0.25) (layer "F.Cu") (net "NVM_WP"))
 (segment (start 21.05 31.25) (end 20.45 31.85) (width 0.25) (layer "F.Cu") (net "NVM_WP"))
 (segment (start 20.45 31.85) (end 20.45 37.55) (width 0.25) (layer "F.Cu") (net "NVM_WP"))
 (segment (start 32.35 32.85) (end 31.35 31.85) (width 0.25) (layer "F.Cu") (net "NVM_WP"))
 (segment (start 22.75 31.85) (end 22.05 31.15) (width 0.25) (layer "F.Cu") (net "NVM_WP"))
 (segment (start 20.45 37.55) (end 18.75 39.25) (width 0.25) (layer "F.Cu") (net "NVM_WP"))
 (segment (start 31.35 31.85) (end 22.75 31.85) (width 0.25) (layer "F.Cu") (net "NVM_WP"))
 (via (at 16.35 29.65) (size 0.6) (drill 0.3) (layers "F.Cu" "B.Cu") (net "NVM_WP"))
 (via (at 20.95 30.15) (size 0.6) (drill 0.3) (layers "F.Cu" "B.Cu") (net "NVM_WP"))
 (segment (start 20.45 29.65) (end 16.35 29.65) (width 0.25) (layer "B.Cu") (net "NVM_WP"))
 (segment (start 20.95 30.15) (end 20.45 29.65) (width 0.25) (layer "B.Cu") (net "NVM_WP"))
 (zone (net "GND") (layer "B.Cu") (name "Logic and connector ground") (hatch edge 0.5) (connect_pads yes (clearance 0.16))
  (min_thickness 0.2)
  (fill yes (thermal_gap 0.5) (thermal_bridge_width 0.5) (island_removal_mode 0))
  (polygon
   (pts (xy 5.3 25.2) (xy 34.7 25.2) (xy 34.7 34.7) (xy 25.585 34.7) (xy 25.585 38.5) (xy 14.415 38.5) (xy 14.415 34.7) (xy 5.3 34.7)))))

